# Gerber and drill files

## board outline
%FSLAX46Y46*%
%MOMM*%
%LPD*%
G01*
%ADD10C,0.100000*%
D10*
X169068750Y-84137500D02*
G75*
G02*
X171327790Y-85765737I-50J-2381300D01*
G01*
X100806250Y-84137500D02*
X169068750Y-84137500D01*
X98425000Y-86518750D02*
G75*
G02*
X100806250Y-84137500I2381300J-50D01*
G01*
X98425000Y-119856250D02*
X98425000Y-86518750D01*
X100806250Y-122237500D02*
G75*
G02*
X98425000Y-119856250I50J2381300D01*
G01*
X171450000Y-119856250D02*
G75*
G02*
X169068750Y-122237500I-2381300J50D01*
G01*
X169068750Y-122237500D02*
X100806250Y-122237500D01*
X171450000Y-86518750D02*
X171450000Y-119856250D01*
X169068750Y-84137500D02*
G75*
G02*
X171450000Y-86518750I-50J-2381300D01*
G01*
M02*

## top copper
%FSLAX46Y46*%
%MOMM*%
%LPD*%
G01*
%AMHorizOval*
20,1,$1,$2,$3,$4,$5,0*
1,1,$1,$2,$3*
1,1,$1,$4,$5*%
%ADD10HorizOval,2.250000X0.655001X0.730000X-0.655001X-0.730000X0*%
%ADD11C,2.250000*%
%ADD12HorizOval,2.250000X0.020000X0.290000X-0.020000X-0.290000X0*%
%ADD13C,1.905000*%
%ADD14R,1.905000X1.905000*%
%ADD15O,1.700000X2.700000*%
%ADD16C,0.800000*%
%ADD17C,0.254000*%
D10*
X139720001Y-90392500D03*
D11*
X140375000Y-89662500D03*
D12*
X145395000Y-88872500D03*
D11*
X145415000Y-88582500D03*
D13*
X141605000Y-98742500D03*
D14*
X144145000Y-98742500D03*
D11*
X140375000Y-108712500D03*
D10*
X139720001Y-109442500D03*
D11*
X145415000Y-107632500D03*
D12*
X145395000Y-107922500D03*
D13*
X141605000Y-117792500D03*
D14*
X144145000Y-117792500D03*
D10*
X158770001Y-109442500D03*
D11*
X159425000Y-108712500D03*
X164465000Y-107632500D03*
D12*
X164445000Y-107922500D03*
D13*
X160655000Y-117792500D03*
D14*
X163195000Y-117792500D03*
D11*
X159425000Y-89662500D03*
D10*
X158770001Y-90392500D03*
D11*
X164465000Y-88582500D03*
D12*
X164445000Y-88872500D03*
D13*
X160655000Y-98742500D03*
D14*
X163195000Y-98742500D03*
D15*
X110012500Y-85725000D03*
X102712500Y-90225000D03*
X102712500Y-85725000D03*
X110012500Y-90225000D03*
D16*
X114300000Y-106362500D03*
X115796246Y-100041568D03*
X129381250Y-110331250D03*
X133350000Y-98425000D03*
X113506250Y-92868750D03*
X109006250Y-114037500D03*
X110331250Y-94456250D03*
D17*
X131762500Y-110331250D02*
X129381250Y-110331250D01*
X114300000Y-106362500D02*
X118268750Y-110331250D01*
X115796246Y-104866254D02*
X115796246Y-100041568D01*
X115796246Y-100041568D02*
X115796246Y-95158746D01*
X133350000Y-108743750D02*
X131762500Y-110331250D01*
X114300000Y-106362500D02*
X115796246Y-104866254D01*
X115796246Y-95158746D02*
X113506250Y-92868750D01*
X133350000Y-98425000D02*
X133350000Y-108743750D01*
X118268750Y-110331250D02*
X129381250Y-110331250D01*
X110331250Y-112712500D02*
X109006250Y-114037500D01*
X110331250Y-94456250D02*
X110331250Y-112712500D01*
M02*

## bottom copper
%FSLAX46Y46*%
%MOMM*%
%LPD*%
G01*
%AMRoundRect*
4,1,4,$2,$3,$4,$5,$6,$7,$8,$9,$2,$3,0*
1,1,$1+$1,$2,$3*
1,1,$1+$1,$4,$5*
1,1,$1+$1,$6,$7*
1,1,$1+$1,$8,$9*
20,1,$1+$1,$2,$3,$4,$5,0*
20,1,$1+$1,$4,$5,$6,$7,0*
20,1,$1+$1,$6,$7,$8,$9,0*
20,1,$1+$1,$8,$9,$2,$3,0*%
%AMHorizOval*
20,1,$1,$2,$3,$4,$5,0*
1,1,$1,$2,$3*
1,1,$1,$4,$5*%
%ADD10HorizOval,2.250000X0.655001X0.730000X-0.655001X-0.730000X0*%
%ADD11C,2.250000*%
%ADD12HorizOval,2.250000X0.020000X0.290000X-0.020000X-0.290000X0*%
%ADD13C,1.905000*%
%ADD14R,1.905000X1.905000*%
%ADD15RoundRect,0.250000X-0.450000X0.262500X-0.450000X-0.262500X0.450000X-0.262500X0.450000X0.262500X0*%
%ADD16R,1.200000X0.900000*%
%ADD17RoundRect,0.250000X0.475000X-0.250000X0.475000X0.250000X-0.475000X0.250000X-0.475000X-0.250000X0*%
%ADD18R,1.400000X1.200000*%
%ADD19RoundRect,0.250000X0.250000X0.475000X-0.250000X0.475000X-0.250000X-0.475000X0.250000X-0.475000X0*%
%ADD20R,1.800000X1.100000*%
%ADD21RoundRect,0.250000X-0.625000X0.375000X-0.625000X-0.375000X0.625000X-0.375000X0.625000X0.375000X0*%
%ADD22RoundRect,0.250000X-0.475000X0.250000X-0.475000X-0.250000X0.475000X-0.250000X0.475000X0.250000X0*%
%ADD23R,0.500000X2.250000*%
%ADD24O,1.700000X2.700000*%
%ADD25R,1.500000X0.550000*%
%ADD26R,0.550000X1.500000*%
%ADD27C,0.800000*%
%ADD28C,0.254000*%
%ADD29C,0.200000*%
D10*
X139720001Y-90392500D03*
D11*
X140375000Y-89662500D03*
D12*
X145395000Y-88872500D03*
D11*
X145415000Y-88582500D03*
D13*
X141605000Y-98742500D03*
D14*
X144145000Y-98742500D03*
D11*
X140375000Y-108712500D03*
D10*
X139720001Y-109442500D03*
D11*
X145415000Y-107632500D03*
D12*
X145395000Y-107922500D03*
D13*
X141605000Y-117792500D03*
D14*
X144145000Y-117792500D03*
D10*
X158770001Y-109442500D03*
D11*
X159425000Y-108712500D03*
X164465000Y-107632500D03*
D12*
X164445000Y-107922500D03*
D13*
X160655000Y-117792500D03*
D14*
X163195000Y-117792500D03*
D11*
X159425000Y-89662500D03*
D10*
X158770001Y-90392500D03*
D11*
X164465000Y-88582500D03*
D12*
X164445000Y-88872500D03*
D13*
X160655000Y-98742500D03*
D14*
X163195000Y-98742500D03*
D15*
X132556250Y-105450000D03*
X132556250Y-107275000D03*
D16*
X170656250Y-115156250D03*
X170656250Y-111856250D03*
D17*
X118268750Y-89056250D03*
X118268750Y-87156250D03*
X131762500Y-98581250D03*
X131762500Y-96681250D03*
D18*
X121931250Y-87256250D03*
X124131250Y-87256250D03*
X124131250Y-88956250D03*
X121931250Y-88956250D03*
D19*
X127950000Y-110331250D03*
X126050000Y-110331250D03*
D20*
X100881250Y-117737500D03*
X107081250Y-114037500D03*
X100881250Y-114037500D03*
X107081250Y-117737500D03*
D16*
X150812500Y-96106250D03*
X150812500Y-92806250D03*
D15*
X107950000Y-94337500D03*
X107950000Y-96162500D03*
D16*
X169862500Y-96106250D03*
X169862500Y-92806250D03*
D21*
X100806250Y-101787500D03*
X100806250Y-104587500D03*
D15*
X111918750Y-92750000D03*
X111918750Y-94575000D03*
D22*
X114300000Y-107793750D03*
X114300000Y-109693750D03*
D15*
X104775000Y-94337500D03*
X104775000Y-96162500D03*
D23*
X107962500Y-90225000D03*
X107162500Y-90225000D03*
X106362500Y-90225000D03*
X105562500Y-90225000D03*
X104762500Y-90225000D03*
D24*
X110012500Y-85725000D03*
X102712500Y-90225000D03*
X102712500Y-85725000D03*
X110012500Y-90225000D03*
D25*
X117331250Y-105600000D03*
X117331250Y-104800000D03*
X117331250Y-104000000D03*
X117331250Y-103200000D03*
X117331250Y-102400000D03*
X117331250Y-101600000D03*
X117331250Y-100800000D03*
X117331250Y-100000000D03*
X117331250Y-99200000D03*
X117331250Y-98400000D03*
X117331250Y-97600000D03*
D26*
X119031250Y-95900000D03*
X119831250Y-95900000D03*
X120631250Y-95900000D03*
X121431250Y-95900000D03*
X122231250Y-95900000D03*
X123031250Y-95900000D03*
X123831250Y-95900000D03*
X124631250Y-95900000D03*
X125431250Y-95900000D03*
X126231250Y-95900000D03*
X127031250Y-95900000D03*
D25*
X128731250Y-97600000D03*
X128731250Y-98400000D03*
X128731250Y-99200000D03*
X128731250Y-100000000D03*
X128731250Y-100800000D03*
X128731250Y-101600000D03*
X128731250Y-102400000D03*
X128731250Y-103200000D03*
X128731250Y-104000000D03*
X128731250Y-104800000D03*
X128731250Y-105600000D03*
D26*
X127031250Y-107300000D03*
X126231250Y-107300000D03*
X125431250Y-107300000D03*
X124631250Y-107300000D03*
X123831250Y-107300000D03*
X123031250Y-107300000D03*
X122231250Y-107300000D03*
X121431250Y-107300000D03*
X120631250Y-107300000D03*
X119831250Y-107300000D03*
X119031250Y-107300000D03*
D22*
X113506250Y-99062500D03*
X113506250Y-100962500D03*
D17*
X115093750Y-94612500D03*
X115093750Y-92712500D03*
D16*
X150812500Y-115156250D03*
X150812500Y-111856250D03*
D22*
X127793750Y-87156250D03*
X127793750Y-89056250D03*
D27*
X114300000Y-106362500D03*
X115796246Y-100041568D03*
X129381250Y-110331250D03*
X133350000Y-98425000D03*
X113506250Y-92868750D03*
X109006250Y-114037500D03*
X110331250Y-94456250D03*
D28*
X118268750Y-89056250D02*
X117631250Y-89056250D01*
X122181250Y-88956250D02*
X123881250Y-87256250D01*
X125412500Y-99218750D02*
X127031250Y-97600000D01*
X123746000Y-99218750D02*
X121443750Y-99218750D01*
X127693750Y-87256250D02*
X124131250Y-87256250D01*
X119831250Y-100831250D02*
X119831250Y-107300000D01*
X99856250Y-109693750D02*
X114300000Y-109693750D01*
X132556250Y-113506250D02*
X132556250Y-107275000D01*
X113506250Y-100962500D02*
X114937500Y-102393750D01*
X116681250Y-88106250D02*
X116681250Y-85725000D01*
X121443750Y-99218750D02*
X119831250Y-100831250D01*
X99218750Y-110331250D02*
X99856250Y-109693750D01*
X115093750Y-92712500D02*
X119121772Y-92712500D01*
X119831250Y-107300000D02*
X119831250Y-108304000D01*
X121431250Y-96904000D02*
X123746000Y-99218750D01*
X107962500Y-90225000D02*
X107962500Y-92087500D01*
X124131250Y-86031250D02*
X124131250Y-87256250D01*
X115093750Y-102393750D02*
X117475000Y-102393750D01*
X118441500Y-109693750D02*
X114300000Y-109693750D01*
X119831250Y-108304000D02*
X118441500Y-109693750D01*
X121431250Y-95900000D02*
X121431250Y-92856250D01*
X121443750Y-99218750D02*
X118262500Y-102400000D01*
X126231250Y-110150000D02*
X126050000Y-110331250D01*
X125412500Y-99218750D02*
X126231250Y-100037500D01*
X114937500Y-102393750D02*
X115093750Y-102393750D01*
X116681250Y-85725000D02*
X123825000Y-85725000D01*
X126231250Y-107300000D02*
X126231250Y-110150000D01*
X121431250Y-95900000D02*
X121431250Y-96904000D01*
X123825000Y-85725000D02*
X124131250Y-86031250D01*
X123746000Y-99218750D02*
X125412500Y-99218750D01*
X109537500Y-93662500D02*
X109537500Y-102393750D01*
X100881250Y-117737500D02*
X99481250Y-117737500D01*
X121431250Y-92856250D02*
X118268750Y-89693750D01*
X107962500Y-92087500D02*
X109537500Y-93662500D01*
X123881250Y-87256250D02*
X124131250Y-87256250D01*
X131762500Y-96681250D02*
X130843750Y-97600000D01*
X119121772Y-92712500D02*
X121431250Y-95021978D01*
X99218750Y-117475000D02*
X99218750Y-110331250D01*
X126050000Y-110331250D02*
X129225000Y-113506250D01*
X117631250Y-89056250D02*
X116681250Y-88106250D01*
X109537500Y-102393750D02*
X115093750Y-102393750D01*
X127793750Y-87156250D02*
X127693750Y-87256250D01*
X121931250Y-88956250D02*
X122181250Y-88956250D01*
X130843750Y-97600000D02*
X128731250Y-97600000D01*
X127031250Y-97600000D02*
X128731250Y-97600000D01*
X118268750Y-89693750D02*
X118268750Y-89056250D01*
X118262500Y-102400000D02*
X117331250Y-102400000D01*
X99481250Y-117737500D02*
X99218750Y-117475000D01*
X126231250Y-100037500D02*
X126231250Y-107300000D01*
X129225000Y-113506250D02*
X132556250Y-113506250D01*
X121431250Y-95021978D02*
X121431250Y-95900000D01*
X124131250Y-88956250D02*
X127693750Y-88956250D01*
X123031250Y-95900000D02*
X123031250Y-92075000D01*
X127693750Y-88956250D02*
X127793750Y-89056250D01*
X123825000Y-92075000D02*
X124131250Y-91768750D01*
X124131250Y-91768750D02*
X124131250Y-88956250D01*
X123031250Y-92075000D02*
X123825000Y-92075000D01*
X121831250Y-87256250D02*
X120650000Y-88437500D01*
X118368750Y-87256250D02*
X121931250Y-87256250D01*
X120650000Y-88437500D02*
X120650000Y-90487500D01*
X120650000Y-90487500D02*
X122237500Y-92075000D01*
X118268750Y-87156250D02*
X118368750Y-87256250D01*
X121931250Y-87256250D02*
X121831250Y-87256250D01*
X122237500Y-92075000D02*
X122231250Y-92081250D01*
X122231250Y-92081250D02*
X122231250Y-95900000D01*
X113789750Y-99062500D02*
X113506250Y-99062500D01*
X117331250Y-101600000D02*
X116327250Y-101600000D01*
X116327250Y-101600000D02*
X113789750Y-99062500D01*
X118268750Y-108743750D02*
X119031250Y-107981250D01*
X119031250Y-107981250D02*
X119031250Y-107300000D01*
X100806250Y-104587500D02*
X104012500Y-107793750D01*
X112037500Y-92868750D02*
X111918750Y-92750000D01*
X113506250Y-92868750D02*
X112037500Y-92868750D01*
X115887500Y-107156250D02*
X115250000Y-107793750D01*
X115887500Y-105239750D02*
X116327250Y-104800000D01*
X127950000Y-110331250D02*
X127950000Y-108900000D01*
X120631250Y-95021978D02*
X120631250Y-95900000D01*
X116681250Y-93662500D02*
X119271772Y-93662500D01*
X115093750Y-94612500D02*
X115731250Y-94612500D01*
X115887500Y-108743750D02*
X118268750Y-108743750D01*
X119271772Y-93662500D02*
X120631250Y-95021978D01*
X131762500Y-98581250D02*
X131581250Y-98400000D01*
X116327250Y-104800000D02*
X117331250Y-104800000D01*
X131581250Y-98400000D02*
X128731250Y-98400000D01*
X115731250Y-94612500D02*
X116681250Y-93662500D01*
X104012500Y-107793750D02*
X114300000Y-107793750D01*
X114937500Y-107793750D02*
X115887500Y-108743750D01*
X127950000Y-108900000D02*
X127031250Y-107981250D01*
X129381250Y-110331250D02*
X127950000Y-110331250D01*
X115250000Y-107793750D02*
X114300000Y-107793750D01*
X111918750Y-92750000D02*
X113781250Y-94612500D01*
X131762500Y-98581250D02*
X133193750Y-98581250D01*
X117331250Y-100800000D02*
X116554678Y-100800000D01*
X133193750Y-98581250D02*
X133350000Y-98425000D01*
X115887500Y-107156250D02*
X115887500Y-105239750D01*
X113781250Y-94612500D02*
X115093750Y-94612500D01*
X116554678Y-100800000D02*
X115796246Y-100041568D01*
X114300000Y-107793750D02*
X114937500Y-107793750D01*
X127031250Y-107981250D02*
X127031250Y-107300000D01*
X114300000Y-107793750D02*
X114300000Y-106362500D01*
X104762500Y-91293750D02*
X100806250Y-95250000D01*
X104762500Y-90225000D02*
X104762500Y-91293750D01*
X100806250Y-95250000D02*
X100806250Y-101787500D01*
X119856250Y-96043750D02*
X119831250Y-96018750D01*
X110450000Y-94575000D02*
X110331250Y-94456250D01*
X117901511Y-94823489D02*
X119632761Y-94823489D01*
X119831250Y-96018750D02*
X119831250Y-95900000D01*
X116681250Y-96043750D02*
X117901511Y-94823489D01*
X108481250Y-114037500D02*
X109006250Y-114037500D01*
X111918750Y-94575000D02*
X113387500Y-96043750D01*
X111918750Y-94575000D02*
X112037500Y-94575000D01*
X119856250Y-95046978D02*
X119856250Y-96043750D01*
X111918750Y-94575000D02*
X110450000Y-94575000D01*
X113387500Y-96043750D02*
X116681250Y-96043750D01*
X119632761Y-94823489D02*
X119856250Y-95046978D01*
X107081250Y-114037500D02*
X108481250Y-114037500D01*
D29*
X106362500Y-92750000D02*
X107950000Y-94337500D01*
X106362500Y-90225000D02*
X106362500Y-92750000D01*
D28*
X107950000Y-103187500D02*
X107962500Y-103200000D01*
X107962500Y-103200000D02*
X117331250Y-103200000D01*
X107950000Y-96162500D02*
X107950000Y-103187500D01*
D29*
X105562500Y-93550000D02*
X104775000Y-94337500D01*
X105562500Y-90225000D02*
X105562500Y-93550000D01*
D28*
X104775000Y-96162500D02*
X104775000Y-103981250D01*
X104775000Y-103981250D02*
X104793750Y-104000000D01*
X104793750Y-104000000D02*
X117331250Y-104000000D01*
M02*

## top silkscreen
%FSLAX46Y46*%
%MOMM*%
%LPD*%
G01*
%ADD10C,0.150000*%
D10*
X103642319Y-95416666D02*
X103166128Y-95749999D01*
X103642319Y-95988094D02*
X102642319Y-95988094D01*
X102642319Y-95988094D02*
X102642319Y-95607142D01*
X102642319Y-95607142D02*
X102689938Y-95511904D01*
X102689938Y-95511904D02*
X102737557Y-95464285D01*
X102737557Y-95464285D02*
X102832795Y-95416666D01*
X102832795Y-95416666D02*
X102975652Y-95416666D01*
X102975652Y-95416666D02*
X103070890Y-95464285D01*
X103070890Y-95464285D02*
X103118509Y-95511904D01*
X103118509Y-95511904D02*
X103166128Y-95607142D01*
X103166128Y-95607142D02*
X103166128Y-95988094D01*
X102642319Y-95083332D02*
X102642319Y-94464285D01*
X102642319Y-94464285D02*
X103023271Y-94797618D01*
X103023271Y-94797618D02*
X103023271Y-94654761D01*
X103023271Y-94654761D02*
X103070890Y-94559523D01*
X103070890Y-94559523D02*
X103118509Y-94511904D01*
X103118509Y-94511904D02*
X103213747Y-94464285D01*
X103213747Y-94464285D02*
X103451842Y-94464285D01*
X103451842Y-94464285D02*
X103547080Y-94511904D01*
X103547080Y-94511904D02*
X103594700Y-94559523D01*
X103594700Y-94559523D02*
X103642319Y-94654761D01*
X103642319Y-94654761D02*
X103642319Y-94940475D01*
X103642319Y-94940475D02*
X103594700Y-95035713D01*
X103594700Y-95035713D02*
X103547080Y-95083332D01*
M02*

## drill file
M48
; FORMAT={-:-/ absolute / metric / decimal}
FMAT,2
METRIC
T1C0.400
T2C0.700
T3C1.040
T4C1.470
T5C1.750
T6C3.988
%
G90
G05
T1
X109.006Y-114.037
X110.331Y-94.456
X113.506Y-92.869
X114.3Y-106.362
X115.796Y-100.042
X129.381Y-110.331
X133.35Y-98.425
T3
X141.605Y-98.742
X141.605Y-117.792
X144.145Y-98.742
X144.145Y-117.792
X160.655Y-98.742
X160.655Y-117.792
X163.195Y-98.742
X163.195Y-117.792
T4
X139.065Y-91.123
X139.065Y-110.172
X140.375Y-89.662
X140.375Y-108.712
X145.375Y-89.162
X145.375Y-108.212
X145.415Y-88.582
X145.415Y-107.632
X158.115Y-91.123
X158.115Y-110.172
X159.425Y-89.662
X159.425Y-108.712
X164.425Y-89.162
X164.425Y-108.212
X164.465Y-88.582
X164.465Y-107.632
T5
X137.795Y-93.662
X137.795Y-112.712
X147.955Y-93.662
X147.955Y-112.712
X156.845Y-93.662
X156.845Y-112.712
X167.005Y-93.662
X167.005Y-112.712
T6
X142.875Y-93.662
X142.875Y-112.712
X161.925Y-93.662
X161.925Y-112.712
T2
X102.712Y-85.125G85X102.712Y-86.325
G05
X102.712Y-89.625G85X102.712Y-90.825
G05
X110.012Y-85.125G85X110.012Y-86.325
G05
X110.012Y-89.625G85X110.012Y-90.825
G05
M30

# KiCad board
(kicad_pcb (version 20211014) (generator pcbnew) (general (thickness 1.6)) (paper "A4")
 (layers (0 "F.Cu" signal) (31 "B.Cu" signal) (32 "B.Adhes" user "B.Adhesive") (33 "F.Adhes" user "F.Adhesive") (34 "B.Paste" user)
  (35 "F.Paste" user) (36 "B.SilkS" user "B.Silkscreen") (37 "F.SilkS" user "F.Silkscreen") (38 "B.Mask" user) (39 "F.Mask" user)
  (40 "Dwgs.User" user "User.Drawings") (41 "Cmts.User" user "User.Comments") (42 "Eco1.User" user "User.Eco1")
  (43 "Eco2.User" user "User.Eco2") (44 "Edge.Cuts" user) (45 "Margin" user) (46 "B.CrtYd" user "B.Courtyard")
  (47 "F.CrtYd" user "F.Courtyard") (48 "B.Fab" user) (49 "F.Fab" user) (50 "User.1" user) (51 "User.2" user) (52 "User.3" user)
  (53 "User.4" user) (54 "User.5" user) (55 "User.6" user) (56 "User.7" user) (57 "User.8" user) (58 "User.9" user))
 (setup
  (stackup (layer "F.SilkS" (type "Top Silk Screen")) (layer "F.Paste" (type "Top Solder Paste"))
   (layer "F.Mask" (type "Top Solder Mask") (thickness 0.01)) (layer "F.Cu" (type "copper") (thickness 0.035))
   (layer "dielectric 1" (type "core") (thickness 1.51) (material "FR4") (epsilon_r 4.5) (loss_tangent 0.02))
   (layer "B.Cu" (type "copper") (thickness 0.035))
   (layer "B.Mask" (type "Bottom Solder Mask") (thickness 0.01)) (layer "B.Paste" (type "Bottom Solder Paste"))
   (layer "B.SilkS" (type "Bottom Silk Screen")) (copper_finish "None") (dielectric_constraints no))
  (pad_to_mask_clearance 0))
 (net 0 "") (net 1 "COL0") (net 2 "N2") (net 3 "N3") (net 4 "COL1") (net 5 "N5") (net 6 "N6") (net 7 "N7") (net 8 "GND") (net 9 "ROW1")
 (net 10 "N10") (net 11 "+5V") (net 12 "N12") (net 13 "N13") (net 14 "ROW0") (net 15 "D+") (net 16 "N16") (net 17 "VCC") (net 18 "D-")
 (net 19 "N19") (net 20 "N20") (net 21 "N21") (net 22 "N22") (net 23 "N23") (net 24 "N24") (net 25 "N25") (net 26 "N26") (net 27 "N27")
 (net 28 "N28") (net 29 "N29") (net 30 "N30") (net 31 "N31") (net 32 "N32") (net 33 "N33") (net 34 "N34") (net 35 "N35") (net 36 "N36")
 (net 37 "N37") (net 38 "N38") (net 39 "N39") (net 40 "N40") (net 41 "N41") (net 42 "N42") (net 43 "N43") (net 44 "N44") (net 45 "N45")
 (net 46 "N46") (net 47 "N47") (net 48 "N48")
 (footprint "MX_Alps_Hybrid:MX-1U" (layer "F.Cu") (at 142.875 93.6625)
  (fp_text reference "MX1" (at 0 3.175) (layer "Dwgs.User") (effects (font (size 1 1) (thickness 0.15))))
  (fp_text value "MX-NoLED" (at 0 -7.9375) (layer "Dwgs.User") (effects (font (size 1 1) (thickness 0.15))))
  (pad "" np_thru_hole circle locked (at 5.08 0 48.0996) (size 1.75 1.75) (drill 1.75) (layers *.Cu *.Mask))
  (pad "" np_thru_hole circle locked (at 0 0) (size 3.9878 3.9878) (drill 3.9878) (layers *.Cu *.Mask))
  (pad "" np_thru_hole circle locked (at -5.08 0 48.0996) (size 1.75 1.75) (drill 1.75) (layers *.Cu *.Mask))
  (pad "1" thru_hole oval locked (at -3.81 -2.54 48.0996) (size 4.211556 2.25) (drill 1.47 (offset 0.980778 0)) (layers *.Cu "B.Mask")
   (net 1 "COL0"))
  (pad "1" thru_hole circle locked (at -2.5 -4) (size 2.25 2.25) (drill 1.47) (layers *.Cu "B.Mask") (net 1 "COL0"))
  (pad "2" thru_hole oval locked (at 2.5 -4.5 86.0548) (size 2.831378 2.25) (drill 1.47 (offset 0.290689 0)) (layers *.Cu "B.Mask")
   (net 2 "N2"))
  (pad "2" thru_hole circle locked (at 2.54 -5.08) (size 2.25 2.25) (drill 1.47) (layers *.Cu "B.Mask") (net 2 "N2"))
  (pad "3" thru_hole circle locked (at -1.27 5.08) (size 1.905 1.905) (drill 1.04) (layers *.Cu "B.Mask"))
  (pad "4" thru_hole rect locked (at 1.27 5.08) (size 1.905 1.905) (drill 1.04) (layers *.Cu "B.Mask")))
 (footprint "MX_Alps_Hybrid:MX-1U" (layer "F.Cu") (at 142.875 112.7125)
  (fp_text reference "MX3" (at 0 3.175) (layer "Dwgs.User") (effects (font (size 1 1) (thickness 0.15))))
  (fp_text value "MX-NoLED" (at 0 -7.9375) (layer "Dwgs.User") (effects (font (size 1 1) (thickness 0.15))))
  (pad "" np_thru_hole circle locked (at -5.08 0 48.0996) (size 1.75 1.75) (drill 1.75) (layers *.Cu *.Mask))
  (pad "" np_thru_hole circle locked (at 0 0) (size 3.9878 3.9878) (drill 3.9878) (layers *.Cu *.Mask))
  (pad "" np_thru_hole circle locked (at 5.08 0 48.0996) (size 1.75 1.75) (drill 1.75) (layers *.Cu *.Mask))
  (pad "1" thru_hole circle locked (at -2.5 -4) (size 2.25 2.25) (drill 1.47) (layers *.Cu "B.Mask") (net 1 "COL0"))
  (pad "1" thru_hole oval locked (at -3.81 -2.54 48.0996) (size 4.211556 2.25) (drill 1.47 (offset 0.980778 0)) (layers *.Cu "B.Mask")
   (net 1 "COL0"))
  (pad "2" thru_hole circle locked (at 2.54 -5.08) (size 2.25 2.25) (drill 1.47) (layers *.Cu "B.Mask") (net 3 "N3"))
  (pad "2" thru_hole oval locked (at 2.5 -4.5 86.0548) (size 2.831378 2.25) (drill 1.47 (offset 0.290689 0)) (layers *.Cu "B.Mask")
   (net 3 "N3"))
  (pad "3" thru_hole circle locked (at -1.27 5.08) (size 1.905 1.905) (drill 1.04) (layers *.Cu "B.Mask"))
  (pad "4" thru_hole rect locked (at 1.27 5.08) (size 1.905 1.905) (drill 1.04) (layers *.Cu "B.Mask")))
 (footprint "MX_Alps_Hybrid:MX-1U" (layer "F.Cu") (at 161.925 112.7125)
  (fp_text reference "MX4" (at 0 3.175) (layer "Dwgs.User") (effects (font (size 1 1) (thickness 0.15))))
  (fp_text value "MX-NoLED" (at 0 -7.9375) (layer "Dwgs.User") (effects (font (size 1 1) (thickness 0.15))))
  (pad "" np_thru_hole circle locked (at 0 0) (size 3.9878 3.9878) (drill 3.9878) (layers *.Cu *.Mask))
  (pad "" np_thru_hole circle locked (at 5.08 0 48.0996) (size 1.75 1.75) (drill 1.75) (layers *.Cu *.Mask))
  (pad "" np_thru_hole circle locked (at -5.08 0 48.0996) (size 1.75 1.75) (drill 1.75) (layers *.Cu *.Mask))
  (pad "1" thru_hole oval locked (at -3.81 -2.54 48.0996) (size 4.211556 2.25) (drill 1.47 (offset 0.980778 0)) (layers *.Cu "B.Mask")
   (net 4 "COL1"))
  (pad "1" thru_hole circle locked (at -2.5 -4) (size 2.25 2.25) (drill 1.47) (layers *.Cu "B.Mask") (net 4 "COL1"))
  (pad "2" thru_hole circle locked (at 2.54 -5.08) (size 2.25 2.25) (drill 1.47) (layers *.Cu "B.Mask") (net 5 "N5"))
  (pad "2" thru_hole oval locked (at 2.5 -4.5 86.0548) (size 2.831378 2.25) (drill 1.47 (offset 0.290689 0)) (layers *.Cu "B.Mask")
   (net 5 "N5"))
  (pad "3" thru_hole circle locked (at -1.27 5.08) (size 1.905 1.905) (drill 1.04) (layers *.Cu "B.Mask"))
  (pad "4" thru_hole rect locked (at 1.27 5.08) (size 1.905 1.905) (drill 1.04) (layers *.Cu "B.Mask")))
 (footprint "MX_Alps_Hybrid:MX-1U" (layer "F.Cu") (at 161.925 93.6625)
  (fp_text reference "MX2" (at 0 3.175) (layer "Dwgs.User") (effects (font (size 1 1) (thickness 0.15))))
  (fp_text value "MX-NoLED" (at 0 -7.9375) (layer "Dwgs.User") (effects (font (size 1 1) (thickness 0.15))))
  (pad "" np_thru_hole circle locked (at 0 0) (size 3.9878 3.9878) (drill 3.9878) (layers *.Cu *.Mask))
  (pad "" np_thru_hole circle locked (at 5.08 0 48.0996) (size 1.75 1.75) (drill 1.75) (layers *.Cu *.Mask))
  (pad "" np_thru_hole circle locked (at -5.08 0 48.0996) (size 1.75 1.75) (drill 1.75) (layers *.Cu *.Mask))
  (pad "1" thru_hole circle locked (at -2.5 -4) (size 2.25 2.25) (drill 1.47) (layers *.Cu "B.Mask") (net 4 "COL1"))
  (pad "1" thru_hole oval locked (at -3.81 -2.54 48.0996) (size 4.211556 2.25) (drill 1.47 (offset 0.980778 0)) (layers *.Cu "B.Mask")
   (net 4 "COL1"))
  (pad "2" thru_hole circle locked (at 2.54 -5.08) (size 2.25 2.25) (drill 1.47) (layers *.Cu "B.Mask") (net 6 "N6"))
  (pad "2" thru_hole oval locked (at 2.5 -4.5 86.0548) (size 2.831378 2.25) (drill 1.47 (offset 0.290689 0)) (layers *.Cu "B.Mask")
   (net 6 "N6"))
  (pad "3" thru_hole circle locked (at -1.27 5.08) (size 1.905 1.905) (drill 1.04) (layers *.Cu "B.Mask"))
  (pad "4" thru_hole rect locked (at 1.27 5.08) (size 1.905 1.905) (drill 1.04) (layers *.Cu "B.Mask")))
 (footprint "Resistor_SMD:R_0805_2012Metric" (layer "B.Cu") (at 132.55625 106.3625 -90)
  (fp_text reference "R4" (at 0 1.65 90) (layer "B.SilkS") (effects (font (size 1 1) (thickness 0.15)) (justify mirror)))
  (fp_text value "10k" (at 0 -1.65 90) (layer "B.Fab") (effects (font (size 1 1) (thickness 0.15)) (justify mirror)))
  (pad "1" smd roundrect (at -0.9125 0 270) (size 1.025 1.4) (layers "B.Cu" "B.Paste" "B.Mask") (roundrect_rratio 0.243902) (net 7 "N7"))
  (pad "2" smd roundrect (at 0.9125 0 270) (size 1.025 1.4) (layers "B.Cu" "B.Paste" "B.Mask") (roundrect_rratio 0.243902) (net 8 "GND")))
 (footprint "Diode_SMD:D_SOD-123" (layer "B.Cu") (at 170.65625 113.50625 90)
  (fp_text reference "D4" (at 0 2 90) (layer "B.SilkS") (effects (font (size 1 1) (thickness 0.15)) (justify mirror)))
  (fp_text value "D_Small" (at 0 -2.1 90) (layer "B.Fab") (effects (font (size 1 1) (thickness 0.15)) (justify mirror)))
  (pad "1" smd rect (at -1.65 0 90) (size 0.9 1.2) (layers "B.Cu" "B.Paste" "B.Mask") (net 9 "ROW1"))
  (pad "2" smd rect (at 1.65 0 90) (size 0.9 1.2) (layers "B.Cu" "B.Paste" "B.Mask") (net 5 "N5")))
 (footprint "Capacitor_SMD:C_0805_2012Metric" (layer "B.Cu") (at 118.26875 88.10625 90)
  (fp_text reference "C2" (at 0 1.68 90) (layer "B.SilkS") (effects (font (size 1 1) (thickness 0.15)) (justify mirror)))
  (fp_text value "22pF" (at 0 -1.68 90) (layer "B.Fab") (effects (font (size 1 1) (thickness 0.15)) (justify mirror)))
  (pad "1" smd roundrect (at -0.95 0 90) (size 1 1.45) (layers "B.Cu" "B.Paste" "B.Mask") (roundrect_rratio 0.25) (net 8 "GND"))
  (pad "2" smd roundrect (at 0.95 0 90) (size 1 1.45) (layers "B.Cu" "B.Paste" "B.Mask") (roundrect_rratio 0.25) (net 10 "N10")))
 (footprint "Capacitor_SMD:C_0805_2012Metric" (layer "B.Cu") (at 131.7625 97.63125 90)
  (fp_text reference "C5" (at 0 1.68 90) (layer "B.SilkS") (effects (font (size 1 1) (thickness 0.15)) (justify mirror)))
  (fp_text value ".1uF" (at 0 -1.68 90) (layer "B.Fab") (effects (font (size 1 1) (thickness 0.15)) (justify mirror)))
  (pad "1" smd roundrect (at -0.95 0 90) (size 1 1.45) (layers "B.Cu" "B.Paste" "B.Mask") (roundrect_rratio 0.25) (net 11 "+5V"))
  (pad "2" smd roundrect (at 0.95 0 90) (size 1 1.45) (layers "B.Cu" "B.Paste" "B.Mask") (roundrect_rratio 0.25) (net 8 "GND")))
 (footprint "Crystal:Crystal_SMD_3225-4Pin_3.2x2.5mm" (layer "B.Cu") (at 123.03125 88.10625)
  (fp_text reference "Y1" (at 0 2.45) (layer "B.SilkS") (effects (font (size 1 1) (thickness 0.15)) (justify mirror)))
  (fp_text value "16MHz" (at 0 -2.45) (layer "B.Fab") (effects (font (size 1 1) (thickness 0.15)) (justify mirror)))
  (pad "1" smd rect (at -1.1 -0.85) (size 1.4 1.2) (layers "B.Cu" "B.Paste" "B.Mask") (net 10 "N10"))
  (pad "2" smd rect (at 1.1 -0.85) (size 1.4 1.2) (layers "B.Cu" "B.Paste" "B.Mask") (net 8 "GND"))
  (pad "3" smd rect (at 1.1 0.85) (size 1.4 1.2) (layers "B.Cu" "B.Paste" "B.Mask") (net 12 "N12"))
  (pad "4" smd rect (at -1.1 0.85) (size 1.4 1.2) (layers "B.Cu" "B.Paste" "B.Mask") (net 8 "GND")))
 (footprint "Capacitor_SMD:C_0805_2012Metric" (layer "B.Cu") (at 127 110.33125 180)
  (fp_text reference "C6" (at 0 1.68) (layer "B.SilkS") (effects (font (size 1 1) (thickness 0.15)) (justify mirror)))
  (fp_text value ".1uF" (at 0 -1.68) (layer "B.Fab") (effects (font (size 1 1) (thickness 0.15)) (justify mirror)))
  (pad "1" smd roundrect (at -0.95 0 180) (size 1 1.45) (layers "B.Cu" "B.Paste" "B.Mask") (roundrect_rratio 0.25) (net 11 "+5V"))
  (pad "2" smd roundrect (at 0.95 0 180) (size 1 1.45) (layers "B.Cu" "B.Paste" "B.Mask") (roundrect_rratio 0.25) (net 8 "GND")))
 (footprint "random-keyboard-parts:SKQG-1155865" (layer "B.Cu") (at 103.98125 115.8875 180)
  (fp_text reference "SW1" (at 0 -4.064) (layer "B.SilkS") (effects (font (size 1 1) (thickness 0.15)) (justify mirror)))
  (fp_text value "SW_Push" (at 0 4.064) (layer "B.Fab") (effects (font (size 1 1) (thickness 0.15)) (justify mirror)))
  (pad "1" smd rect locked (at 3.1 -1.85 180) (size 1.8 1.1) (layers "B.Cu" "B.Paste" "B.Mask") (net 8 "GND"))
  (pad "2" smd rect locked (at -3.1 1.85 180) (size 1.8 1.1) (layers "B.Cu" "B.Paste" "B.Mask") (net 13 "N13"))
  (pad "3" smd rect locked (at 3.1 1.85 180) (size 1.8 1.1) (layers "B.Cu" "B.Paste" "B.Mask"))
  (pad "4" smd rect locked (at -3.1 -1.85 180) (size 1.8 1.1) (layers "B.Cu" "B.Paste" "B.Mask")))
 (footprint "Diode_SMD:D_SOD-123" (layer "B.Cu") (at 150.8125 94.45625 90)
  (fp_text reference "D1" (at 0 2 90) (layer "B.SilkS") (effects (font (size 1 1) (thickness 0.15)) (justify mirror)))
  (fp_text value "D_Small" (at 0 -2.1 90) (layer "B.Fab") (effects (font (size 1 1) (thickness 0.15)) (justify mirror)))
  (pad "1" smd rect (at -1.65 0 90) (size 0.9 1.2) (layers "B.Cu" "B.Paste" "B.Mask") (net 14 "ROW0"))
  (pad "2" smd rect (at 1.65 0 90) (size 0.9 1.2) (layers "B.Cu" "B.Paste" "B.Mask") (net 2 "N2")))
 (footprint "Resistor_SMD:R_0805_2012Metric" (layer "B.Cu") (at 107.95 95.25 -90)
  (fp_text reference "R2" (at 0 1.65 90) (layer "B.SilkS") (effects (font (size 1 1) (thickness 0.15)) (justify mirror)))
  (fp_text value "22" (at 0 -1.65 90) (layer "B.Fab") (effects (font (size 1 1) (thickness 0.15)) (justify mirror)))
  (pad "1" smd roundrect (at -0.9125 0 270) (size 1.025 1.4) (layers "B.Cu" "B.Paste" "B.Mask") (roundrect_rratio 0.243902) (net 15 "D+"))
  (pad "2" smd roundrect (at 0.9125 0 270) (size 1.025 1.4) (layers "B.Cu" "B.Paste" "B.Mask") (roundrect_rratio 0.243902) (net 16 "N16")))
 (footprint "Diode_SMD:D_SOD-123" (layer "B.Cu") (at 169.8625 94.45625 90)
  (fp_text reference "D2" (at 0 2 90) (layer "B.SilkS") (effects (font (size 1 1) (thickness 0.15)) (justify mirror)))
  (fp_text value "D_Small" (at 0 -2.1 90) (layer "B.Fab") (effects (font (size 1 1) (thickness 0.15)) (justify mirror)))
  (pad "1" smd rect (at -1.65 0 90) (size 0.9 1.2) (layers "B.Cu" "B.Paste" "B.Mask") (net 14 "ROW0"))
  (pad "2" smd rect (at 1.65 0 90) (size 0.9 1.2) (layers "B.Cu" "B.Paste" "B.Mask") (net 6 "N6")))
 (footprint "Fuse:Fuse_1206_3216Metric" (layer "B.Cu") (at 100.80625 103.1875 -90)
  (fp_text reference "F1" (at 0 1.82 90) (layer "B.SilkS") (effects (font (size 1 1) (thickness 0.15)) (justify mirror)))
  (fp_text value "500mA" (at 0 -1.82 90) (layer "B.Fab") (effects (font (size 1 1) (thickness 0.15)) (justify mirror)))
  (pad "1" smd roundrect (at -1.4 0 270) (size 1.25 1.75) (layers "B.Cu" "B.Paste" "B.Mask") (roundrect_rratio 0.2) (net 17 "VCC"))
  (pad "2" smd roundrect (at 1.4 0 270) (size 1.25 1.75) (layers "B.Cu" "B.Paste" "B.Mask") (roundrect_rratio 0.2) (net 11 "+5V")))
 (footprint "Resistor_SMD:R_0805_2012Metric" (layer "B.Cu") (at 111.91875 93.6625 -90)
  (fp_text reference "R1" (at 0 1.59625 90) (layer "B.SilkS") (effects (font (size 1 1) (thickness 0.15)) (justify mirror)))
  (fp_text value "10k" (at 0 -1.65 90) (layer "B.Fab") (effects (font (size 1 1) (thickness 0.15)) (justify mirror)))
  (pad "1" smd roundrect (at -0.9125 0 270) (size 1.025 1.4) (layers "B.Cu" "B.Paste" "B.Mask") (roundrect_rratio 0.243902) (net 11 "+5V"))
  (pad "2" smd roundrect (at 0.9125 0 270) (size 1.025 1.4) (layers "B.Cu" "B.Paste" "B.Mask") (roundrect_rratio 0.243902) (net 13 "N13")))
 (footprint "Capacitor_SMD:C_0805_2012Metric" (layer "B.Cu") (at 114.3 108.74375 -90)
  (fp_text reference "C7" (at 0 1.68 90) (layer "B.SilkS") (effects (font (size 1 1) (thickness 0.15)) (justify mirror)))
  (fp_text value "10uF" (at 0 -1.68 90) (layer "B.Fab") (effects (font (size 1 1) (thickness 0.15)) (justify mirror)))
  (pad "1" smd roundrect (at -0.95 0 270) (size 1 1.45) (layers "B.Cu" "B.Paste" "B.Mask") (roundrect_rratio 0.25) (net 11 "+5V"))
  (pad "2" smd roundrect (at 0.95 0 270) (size 1 1.45) (layers "B.Cu" "B.Paste" "B.Mask") (roundrect_rratio 0.25) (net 8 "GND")))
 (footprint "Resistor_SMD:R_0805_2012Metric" (layer "B.Cu") (at 104.775 95.25 -90)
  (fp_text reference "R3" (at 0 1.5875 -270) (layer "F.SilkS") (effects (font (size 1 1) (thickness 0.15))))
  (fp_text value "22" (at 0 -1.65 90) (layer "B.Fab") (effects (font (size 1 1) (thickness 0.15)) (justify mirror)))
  (pad "1" smd roundrect (at -0.9125 0 270) (size 1.025 1.4) (layers "B.Cu" "B.Paste" "B.Mask") (roundrect_rratio 0.243902) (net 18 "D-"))
  (pad "2" smd roundrect (at 0.9125 0 270) (size 1.025 1.4) (layers "B.Cu" "B.Paste" "B.Mask") (roundrect_rratio 0.243902) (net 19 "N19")))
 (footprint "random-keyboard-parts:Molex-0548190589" (layer "B.Cu") (at 106.3625 85.725 -90)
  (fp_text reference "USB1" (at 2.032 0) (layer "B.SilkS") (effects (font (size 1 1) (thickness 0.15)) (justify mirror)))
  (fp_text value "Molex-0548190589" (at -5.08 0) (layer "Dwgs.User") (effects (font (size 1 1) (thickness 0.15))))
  (pad "1" smd rect locked (at 4.5 -1.6 270) (size 2.25 0.5) (layers "B.Cu" "B.Paste" "B.Mask") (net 8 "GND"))
  (pad "2" smd rect locked (at 4.5 -0.8 270) (size 2.25 0.5) (layers "B.Cu" "B.Paste" "B.Mask") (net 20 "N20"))
  (pad "3" smd rect locked (at 4.5 0 270) (size 2.25 0.5) (layers "B.Cu" "B.Paste" "B.Mask") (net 15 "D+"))
  (pad "4" smd rect locked (at 4.5 0.8 270) (size 2.25 0.5) (layers "B.Cu" "B.Paste" "B.Mask") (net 18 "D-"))
  (pad "5" smd rect locked (at 4.5 1.6 270) (size 2.25 0.5) (layers "B.Cu" "B.Paste" "B.Mask") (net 17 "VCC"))
  (pad "6" thru_hole oval locked (at 0 -3.65 270) (size 2.7 1.7) (drill oval 1.9 0.7) (layers *.Cu *.Mask) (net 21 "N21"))
  (pad "6" thru_hole oval locked (at 4.5 3.65 270) (size 2.7 1.7) (drill oval 1.9 0.7) (layers *.Cu *.Mask) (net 21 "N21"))
  (pad "6" thru_hole oval locked (at 0 3.65 270) (size 2.7 1.7) (drill oval 1.9 0.7) (layers *.Cu *.Mask) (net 21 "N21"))
  (pad "6" thru_hole oval locked (at 4.5 -3.65 270) (size 2.7 1.7) (drill oval 1.9 0.7) (layers *.Cu *.Mask) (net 21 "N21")))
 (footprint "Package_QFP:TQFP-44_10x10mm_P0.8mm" (layer "B.Cu") (at 123.03125 101.6)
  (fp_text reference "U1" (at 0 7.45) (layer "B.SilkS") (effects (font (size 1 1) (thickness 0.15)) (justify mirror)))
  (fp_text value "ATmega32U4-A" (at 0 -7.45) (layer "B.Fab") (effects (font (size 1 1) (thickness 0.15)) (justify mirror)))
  (pad "1" smd rect (at -5.7 4) (size 1.5 0.55) (layers "B.Cu" "B.Paste" "B.Mask") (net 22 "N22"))
  (pad "2" smd rect (at -5.7 3.2) (size 1.5 0.55) (layers "B.Cu" "B.Paste" "B.Mask") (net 11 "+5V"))
  (pad "3" smd rect (at -5.7 2.4) (size 1.5 0.55) (layers "B.Cu" "B.Paste" "B.Mask") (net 19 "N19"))
  (pad "4" smd rect (at -5.7 1.6) (size 1.5 0.55) (layers "B.Cu" "B.Paste" "B.Mask") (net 16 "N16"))
  (pad "5" smd rect (at -5.7 0.8) (size 1.5 0.55) (layers "B.Cu" "B.Paste" "B.Mask") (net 8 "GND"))
  (pad "6" smd rect (at -5.7 0) (size 1.5 0.55) (layers "B.Cu" "B.Paste" "B.Mask") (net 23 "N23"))
  (pad "7" smd rect (at -5.7 -0.8) (size 1.5 0.55) (layers "B.Cu" "B.Paste" "B.Mask") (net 11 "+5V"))
  (pad "8" smd rect (at -5.7 -1.6) (size 1.5 0.55) (layers "B.Cu" "B.Paste" "B.Mask") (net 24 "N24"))
  (pad "9" smd rect (at -5.7 -2.4) (size 1.5 0.55) (layers "B.Cu" "B.Paste" "B.Mask") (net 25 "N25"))
  (pad "10" smd rect (at -5.7 -3.2) (size 1.5 0.55) (layers "B.Cu" "B.Paste" "B.Mask") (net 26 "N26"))
  (pad "11" smd rect (at -5.7 -4) (size 1.5 0.55) (layers "B.Cu" "B.Paste" "B.Mask") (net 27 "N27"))
  (pad "12" smd rect (at -4 -5.7 270) (size 1.5 0.55) (layers "B.Cu" "B.Paste" "B.Mask") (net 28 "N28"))
  (pad "13" smd rect (at -3.2 -5.7 270) (size 1.5 0.55) (layers "B.Cu" "B.Paste" "B.Mask") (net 13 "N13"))
  (pad "14" smd rect (at -2.4 -5.7 270) (size 1.5 0.55) (layers "B.Cu" "B.Paste" "B.Mask") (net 11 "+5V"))
  (pad "15" smd rect (at -1.6 -5.7 270) (size 1.5 0.55) (layers "B.Cu" "B.Paste" "B.Mask") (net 8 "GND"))
  (pad "16" smd rect (at -0.8 -5.7 270) (size 1.5 0.55) (layers "B.Cu" "B.Paste" "B.Mask") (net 10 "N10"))
  (pad "17" smd rect (at 0 -5.7 270) (size 1.5 0.55) (layers "B.Cu" "B.Paste" "B.Mask") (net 12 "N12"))
  (pad "18" smd rect (at 0.8 -5.7 270) (size 1.5 0.55) (layers "B.Cu" "B.Paste" "B.Mask") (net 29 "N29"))
  (pad "19" smd rect (at 1.6 -5.7 270) (size 1.5 0.55) (layers "B.Cu" "B.Paste" "B.Mask") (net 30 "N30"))
  (pad "20" smd rect (at 2.4 -5.7 270) (size 1.5 0.55) (layers "B.Cu" "B.Paste" "B.Mask") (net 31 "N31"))
  (pad "21" smd rect (at 3.2 -5.7 270) (size 1.5 0.55) (layers "B.Cu" "B.Paste" "B.Mask") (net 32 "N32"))
  (pad "22" smd rect (at 4 -5.7 270) (size 1.5 0.55) (layers "B.Cu" "B.Paste" "B.Mask") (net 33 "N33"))
  (pad "23" smd rect (at 5.7 -4) (size 1.5 0.55) (layers "B.Cu" "B.Paste" "B.Mask") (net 8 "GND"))
  (pad "24" smd rect (at 5.7 -3.2) (size 1.5 0.55) (layers "B.Cu" "B.Paste" "B.Mask") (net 11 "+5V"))
  (pad "25" smd rect (at 5.7 -2.4) (size 1.5 0.55) (layers "B.Cu" "B.Paste" "B.Mask") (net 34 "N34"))
  (pad "26" smd rect (at 5.7 -1.6) (size 1.5 0.55) (layers "B.Cu" "B.Paste" "B.Mask") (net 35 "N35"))
  (pad "27" smd rect (at 5.7 -0.8) (size 1.5 0.55) (layers "B.Cu" "B.Paste" "B.Mask") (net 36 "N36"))
  (pad "28" smd rect (at 5.7 0) (size 1.5 0.55) (layers "B.Cu" "B.Paste" "B.Mask") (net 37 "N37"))
  (pad "29" smd rect (at 5.7 0.8) (size 1.5 0.55) (layers "B.Cu" "B.Paste" "B.Mask") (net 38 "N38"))
  (pad "30" smd rect (at 5.7 1.6) (size 1.5 0.55) (layers "B.Cu" "B.Paste" "B.Mask") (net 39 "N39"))
  (pad "31" smd rect (at 5.7 2.4) (size 1.5 0.55) (layers "B.Cu" "B.Paste" "B.Mask") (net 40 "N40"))
  (pad "32" smd rect (at 5.7 3.2) (size 1.5 0.55) (layers "B.Cu" "B.Paste" "B.Mask") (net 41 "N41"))
  (pad "33" smd rect (at 5.7 4) (size 1.5 0.55) (layers "B.Cu" "B.Paste" "B.Mask") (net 7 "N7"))
  (pad "34" smd rect (at 4 5.7 270) (size 1.5 0.55) (layers "B.Cu" "B.Paste" "B.Mask") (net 11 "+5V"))
  (pad "35" smd rect (at 3.2 5.7 270) (size 1.5 0.55) (layers "B.Cu" "B.Paste" "B.Mask") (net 8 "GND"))
  (pad "36" smd rect (at 2.4 5.7 270) (size 1.5 0.55) (layers "B.Cu" "B.Paste" "B.Mask") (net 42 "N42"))
  (pad "37" smd rect (at 1.6 5.7 270) (size 1.5 0.55) (layers "B.Cu" "B.Paste" "B.Mask") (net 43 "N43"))
  (pad "38" smd rect (at 0.8 5.7 270) (size 1.5 0.55) (layers "B.Cu" "B.Paste" "B.Mask") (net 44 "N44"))
  (pad "39" smd rect (at 0 5.7 270) (size 1.5 0.55) (layers "B.Cu" "B.Paste" "B.Mask") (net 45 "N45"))
  (pad "40" smd rect (at -0.8 5.7 270) (size 1.5 0.55) (layers "B.Cu" "B.Paste" "B.Mask") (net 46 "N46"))
  (pad "41" smd rect (at -1.6 5.7 270) (size 1.5 0.55) (layers "B.Cu" "B.Paste" "B.Mask") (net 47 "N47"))
  (pad "42" smd rect (at -2.4 5.7 270) (size 1.5 0.55) (layers "B.Cu" "B.Paste" "B.Mask") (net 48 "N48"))
  (pad "43" smd rect (at -3.2 5.7 270) (size 1.5 0.55) (layers "B.Cu" "B.Paste" "B.Mask") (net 8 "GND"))
  (pad "44" smd rect (at -4 5.7 270) (size 1.5 0.55) (layers "B.Cu" "B.Paste" "B.Mask") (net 11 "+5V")))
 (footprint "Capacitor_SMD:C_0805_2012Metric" (layer "B.Cu") (at 113.50625 100.0125 -90)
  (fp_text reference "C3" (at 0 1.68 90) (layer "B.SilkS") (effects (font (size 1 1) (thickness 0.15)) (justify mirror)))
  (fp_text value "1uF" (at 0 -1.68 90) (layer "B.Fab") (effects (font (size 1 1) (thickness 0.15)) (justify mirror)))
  (pad "1" smd roundrect (at -0.95 0 270) (size 1 1.45) (layers "B.Cu" "B.Paste" "B.Mask") (roundrect_rratio 0.25) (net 23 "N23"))
  (pad "2" smd roundrect (at 0.95 0 270) (size 1 1.45) (layers "B.Cu" "B.Paste" "B.Mask") (roundrect_rratio 0.25) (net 8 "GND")))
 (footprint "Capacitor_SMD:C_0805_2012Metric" (layer "B.Cu") (at 115.09375 93.6625 90)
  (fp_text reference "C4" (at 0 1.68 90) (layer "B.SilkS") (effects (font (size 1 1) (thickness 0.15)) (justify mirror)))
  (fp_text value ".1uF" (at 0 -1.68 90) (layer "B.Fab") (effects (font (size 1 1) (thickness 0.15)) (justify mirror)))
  (pad "1" smd roundrect (at -0.95 0 90) (size 1 1.45) (layers "B.Cu" "B.Paste" "B.Mask") (roundrect_rratio 0.25) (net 11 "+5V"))
  (pad "2" smd roundrect (at 0.95 0 90) (size 1 1.45) (layers "B.Cu" "B.Paste" "B.Mask") (roundrect_rratio 0.25) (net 8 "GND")))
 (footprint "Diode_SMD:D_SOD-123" (layer "B.Cu") (at 150.8125 113.50625 90)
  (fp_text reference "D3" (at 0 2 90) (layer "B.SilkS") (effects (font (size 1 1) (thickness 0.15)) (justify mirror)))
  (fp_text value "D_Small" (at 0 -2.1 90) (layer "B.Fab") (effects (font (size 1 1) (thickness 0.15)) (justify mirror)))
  (pad "1" smd rect (at -1.65 0 90) (size 0.9 1.2) (layers "B.Cu" "B.Paste" "B.Mask") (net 9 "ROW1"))
  (pad "2" smd rect (at 1.65 0 90) (size 0.9 1.2) (layers "B.Cu" "B.Paste" "B.Mask") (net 3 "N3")))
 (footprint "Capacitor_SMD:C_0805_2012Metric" (layer "B.Cu") (at 127.79375 88.10625 -90)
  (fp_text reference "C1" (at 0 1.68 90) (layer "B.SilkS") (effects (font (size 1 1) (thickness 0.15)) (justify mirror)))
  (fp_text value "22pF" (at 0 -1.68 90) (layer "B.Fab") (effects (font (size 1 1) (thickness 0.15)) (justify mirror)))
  (pad "1" smd roundrect (at -0.95 0 270) (size 1 1.45) (layers "B.Cu" "B.Paste" "B.Mask") (roundrect_rratio 0.25) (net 8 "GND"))
  (pad "2" smd roundrect (at 0.95 0 270) (size 1 1.45) (layers "B.Cu" "B.Paste" "B.Mask") (roundrect_rratio 0.25) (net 12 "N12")))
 (gr_arc (start 169.06875 84.1375) (mid 170.461091 84.58698) (end 171.327802 85.765733) (layer "Edge.Cuts") (width 0.1))
 (gr_line (start 100.80625 84.1375) (end 169.06875 84.1375) (layer "Edge.Cuts") (width 0.1))
 (gr_arc (start 98.425 86.51875) (mid 99.122452 84.834952) (end 100.80625 84.1375) (layer "Edge.Cuts") (width 0.1))
 (gr_line (start 98.425 119.85625) (end 98.425 86.51875) (layer "Edge.Cuts") (width 0.1))
 (gr_arc (start 100.80625 122.2375) (mid 99.122452 121.540048) (end 98.425 119.85625) (layer "Edge.Cuts") (width 0.1))
 (gr_arc (start 171.45 119.85625) (mid 170.752548 121.540048) (end 169.06875 122.2375) (layer "Edge.Cuts") (width 0.1))
 (gr_line (start 169.06875 122.2375) (end 100.80625 122.2375) (layer "Edge.Cuts") (width 0.1))
 (gr_line (start 171.45 86.51875) (end 171.45 119.85625) (layer "Edge.Cuts") (width 0.1))
 (gr_arc (start 169.06875 84.1375) (mid 170.752548 84.834952) (end 171.45 86.51875) (layer "Edge.Cuts") (width 0.1))
 (segment (start 118.26875 89.05625) (end 117.63125 89.05625) (width 0.254) (layer "B.Cu") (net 8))
 (segment (start 122.18125 88.95625) (end 123.88125 87.25625) (width 0.254) (layer "B.Cu") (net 8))
 (segment (start 125.4125 99.21875) (end 127.03125 97.6) (width 0.254) (layer "B.Cu") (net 8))
 (segment (start 123.746 99.21875) (end 121.44375 99.21875) (width 0.254) (layer "B.Cu") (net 8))
 (segment (start 127.69375 87.25625) (end 124.13125 87.25625) (width 0.254) (layer "B.Cu") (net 8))
 (segment (start 119.83125 100.83125) (end 119.83125 107.3) (width 0.254) (layer "B.Cu") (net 8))
 (segment (start 99.85625 109.69375) (end 114.3 109.69375) (width 0.254) (layer "B.Cu") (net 8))
 (segment (start 132.55625 113.50625) (end 132.55625 107.275) (width 0.254) (layer "B.Cu") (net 8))
 (segment (start 113.50625 100.9625) (end 114.9375 102.39375) (width 0.254) (layer "B.Cu") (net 8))
 (segment (start 116.68125 88.10625) (end 116.68125 85.725) (width 0.254) (layer "B.Cu") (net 8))
 (segment (start 121.44375 99.21875) (end 119.83125 100.83125) (width 0.254) (layer "B.Cu") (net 8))
 (segment (start 99.21875 110.33125) (end 99.85625 109.69375) (width 0.254) (layer "B.Cu") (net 8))
 (segment (start 115.09375 92.7125) (end 119.121772 92.7125) (width 0.254) (layer "B.Cu") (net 8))
 (segment (start 119.83125 107.3) (end 119.83125 108.304) (width 0.254) (layer "B.Cu") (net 8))
 (segment (start 121.43125 96.904) (end 123.746 99.21875) (width 0.254) (layer "B.Cu") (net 8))
 (segment (start 107.9625 90.225) (end 107.9625 92.0875) (width 0.254) (layer "B.Cu") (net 8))
 (segment (start 124.13125 86.03125) (end 124.13125 87.25625) (width 0.254) (layer "B.Cu") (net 8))
 (segment (start 115.09375 102.39375) (end 117.475 102.39375) (width 0.254) (layer "B.Cu") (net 8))
 (segment (start 118.4415 109.69375) (end 114.3 109.69375) (width 0.254) (layer "B.Cu") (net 8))
 (segment (start 119.83125 108.304) (end 118.4415 109.69375) (width 0.254) (layer "B.Cu") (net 8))
 (segment (start 121.43125 95.9) (end 121.43125 92.85625) (width 0.254) (layer "B.Cu") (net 8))
 (segment (start 121.44375 99.21875) (end 118.2625 102.4) (width 0.254) (layer "B.Cu") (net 8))
 (segment (start 126.23125 110.15) (end 126.05 110.33125) (width 0.254) (layer "B.Cu") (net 8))
 (segment (start 125.4125 99.21875) (end 126.23125 100.0375) (width 0.254) (layer "B.Cu") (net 8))
 (segment (start 114.9375 102.39375) (end 115.09375 102.39375) (width 0.254) (layer "B.Cu") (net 8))
 (segment (start 116.68125 85.725) (end 123.825 85.725) (width 0.254) (layer "B.Cu") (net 8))
 (segment (start 126.23125 107.3) (end 126.23125 110.15) (width 0.254) (layer "B.Cu") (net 8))
 (segment (start 121.43125 95.9) (end 121.43125 96.904) (width 0.254) (layer "B.Cu") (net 8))
 (segment (start 123.825 85.725) (end 124.13125 86.03125) (width 0.254) (layer "B.Cu") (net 8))
 (segment (start 123.746 99.21875) (end 125.4125 99.21875) (width 0.254) (layer "B.Cu") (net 8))
 (segment (start 109.5375 93.6625) (end 109.5375 102.39375) (width 0.254) (layer "B.Cu") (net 8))
 (segment (start 100.88125 117.7375) (end 99.48125 117.7375) (width 0.254) (layer "B.Cu") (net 8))
 (segment (start 121.43125 92.85625) (end 118.26875 89.69375) (width 0.254) (layer "B.Cu") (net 8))
 (segment (start 107.9625 92.0875) (end 109.5375 93.6625) (width 0.254) (layer "B.Cu") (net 8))
 (segment (start 123.88125 87.25625) (end 124.13125 87.25625) (width 0.254) (layer "B.Cu") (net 8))
 (segment (start 131.7625 96.68125) (end 130.84375 97.6) (width 0.254) (layer "B.Cu") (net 8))
 (segment (start 119.121772 92.7125) (end 121.43125 95.021978) (width 0.254) (layer "B.Cu") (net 8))
 (segment (start 99.21875 117.475) (end 99.21875 110.33125) (width 0.254) (layer "B.Cu") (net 8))
 (segment (start 126.05 110.33125) (end 129.225 113.50625) (width 0.254) (layer "B.Cu") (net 8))
 (segment (start 117.63125 89.05625) (end 116.68125 88.10625) (width 0.254) (layer "B.Cu") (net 8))
 (segment (start 109.5375 102.39375) (end 115.09375 102.39375) (width 0.254) (layer "B.Cu") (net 8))
 (segment (start 127.79375 87.15625) (end 127.69375 87.25625) (width 0.254) (layer "B.Cu") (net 8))
 (segment (start 121.93125 88.95625) (end 122.18125 88.95625) (width 0.254) (layer "B.Cu") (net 8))
 (segment (start 130.84375 97.6) (end 128.73125 97.6) (width 0.254) (layer "B.Cu") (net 8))
 (segment (start 127.03125 97.6) (end 128.73125 97.6) (width 0.254) (layer "B.Cu") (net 8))
 (segment (start 118.26875 89.69375) (end 118.26875 89.05625) (width 0.254) (layer "B.Cu") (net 8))
 (segment (start 118.2625 102.4) (end 117.33125 102.4) (width 0.254) (layer "B.Cu") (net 8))
 (segment (start 99.48125 117.7375) (end 99.21875 117.475) (width 0.254) (layer "B.Cu") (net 8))
 (segment (start 126.23125 100.0375) (end 126.23125 107.3) (width 0.254) (layer "B.Cu") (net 8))
 (segment (start 129.225 113.50625) (end 132.55625 113.50625) (width 0.254) (layer "B.Cu") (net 8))
 (segment (start 121.43125 95.021978) (end 121.43125 95.9) (width 0.254) (layer "B.Cu") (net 8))
 (segment (start 124.13125 88.95625) (end 127.69375 88.95625) (width 0.254) (layer "B.Cu") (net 12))
 (segment (start 123.03125 95.9) (end 123.03125 92.075) (width 0.254) (layer "B.Cu") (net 12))
 (segment (start 127.69375 88.95625) (end 127.79375 89.05625) (width 0.254) (layer "B.Cu") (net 12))
 (segment (start 123.825 92.075) (end 124.13125 91.76875) (width 0.254) (layer "B.Cu") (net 12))
 (segment (start 124.13125 91.76875) (end 124.13125 88.95625) (width 0.254) (layer "B.Cu") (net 12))
 (segment (start 123.03125 92.075) (end 123.825 92.075) (width 0.254) (layer "B.Cu") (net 12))
 (segment (start 121.83125 87.25625) (end 120.65 88.4375) (width 0.254) (layer "B.Cu") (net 10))
 (segment (start 118.36875 87.25625) (end 121.93125 87.25625) (width 0.254) (layer "B.Cu") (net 10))
 (segment (start 120.65 88.4375) (end 120.65 90.4875) (width 0.254) (layer "B.Cu") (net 10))
 (segment (start 120.65 90.4875) (end 122.2375 92.075) (width 0.254) (layer "B.Cu") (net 10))
 (segment (start 118.26875 87.15625) (end 118.36875 87.25625) (width 0.254) (layer "B.Cu") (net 10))
 (segment (start 121.93125 87.25625) (end 121.83125 87.25625) (width 0.254) (layer "B.Cu") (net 10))
 (segment (start 122.2375 92.075) (end 122.23125 92.08125) (width 0.254) (layer "B.Cu") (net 10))
 (segment (start 122.23125 92.08125) (end 122.23125 95.9) (width 0.254) (layer "B.Cu") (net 10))
 (segment (start 113.78975 99.0625) (end 113.50625 99.0625) (width 0.254) (layer "B.Cu") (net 23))
 (segment (start 117.33125 101.6) (end 116.32725 101.6) (width 0.254) (layer "B.Cu") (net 23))
 (segment (start 116.32725 101.6) (end 113.78975 99.0625) (width 0.254) (layer "B.Cu") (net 23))
 (segment (start 131.7625 110.33125) (end 129.38125 110.33125) (width 0.254) (layer "F.Cu") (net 11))
 (segment (start 114.3 106.3625) (end 118.26875 110.33125) (width 0.254) (layer "F.Cu") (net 11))
 (segment (start 115.796246 104.866254) (end 115.796246 100.041568) (width 0.254) (layer "F.Cu") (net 11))
 (segment (start 115.796246 100.041568) (end 115.796246 95.158746) (width 0.254) (layer "F.Cu") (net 11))
 (segment (start 133.35 108.74375) (end 131.7625 110.33125) (width 0.254) (layer "F.Cu") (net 11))
 (segment (start 114.3 106.3625) (end 115.796246 104.866254) (width 0.254) (layer "F.Cu") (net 11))
 (segment (start 115.796246 95.158746) (end 113.50625 92.86875) (width 0.254) (layer "F.Cu") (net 11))
 (segment (start 133.35 98.425) (end 133.35 108.74375) (width 0.254) (layer "F.Cu") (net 11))
 (segment (start 118.26875 110.33125) (end 129.38125 110.33125) (width 0.254) (layer "F.Cu") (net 11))
 (via (at 114.3 106.3625) (size 0.8) (drill 0.4) (layers "F.Cu" "B.Cu") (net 11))
 (via (at 115.796246 100.041568) (size 0.8) (drill 0.4) (layers "F.Cu" "B.Cu") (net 11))
 (via (at 129.38125 110.33125) (size 0.8) (drill 0.4) (layers "F.Cu" "B.Cu") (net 11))
 (via (at 133.35 98.425) (size 0.8) (drill 0.4) (layers "F.Cu" "B.Cu") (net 11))
 (via (at 113.50625 92.86875) (size 0.8) (drill 0.4) (layers "F.Cu" "B.Cu") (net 11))
 (segment (start 118.26875 108.74375) (end 119.03125 107.98125) (width 0.254) (layer "B.Cu") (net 11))
 (segment (start 119.03125 107.98125) (end 119.03125 107.3) (width 0.254) (layer "B.Cu") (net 11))
 (segment (start 100.80625 104.5875) (end 104.0125 107.79375) (width 0.254) (layer "B.Cu") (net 11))
 (segment (start 112.0375 92.86875) (end 111.91875 92.75) (width 0.254) (layer "B.Cu") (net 11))
 (segment (start 113.50625 92.86875) (end 112.0375 92.86875) (width 0.254) (layer "B.Cu") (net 11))
 (segment (start 115.8875 107.15625) (end 115.25 107.79375) (width 0.254) (layer "B.Cu") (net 11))
 (segment (start 115.8875 105.23975) (end 116.32725 104.8) (width 0.254) (layer "B.Cu") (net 11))
 (segment (start 127.95 110.33125) (end 127.95 108.9) (width 0.254) (layer "B.Cu") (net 11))
 (segment (start 120.63125 95.021978) (end 120.63125 95.9) (width 0.254) (layer "B.Cu") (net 11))
 (segment (start 116.68125 93.6625) (end 119.271772 93.6625) (width 0.254) (layer "B.Cu") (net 11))
 (segment (start 115.09375 94.6125) (end 115.73125 94.6125) (width 0.254) (layer "B.Cu") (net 11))
 (segment (start 115.8875 108.74375) (end 118.26875 108.74375) (width 0.254) (layer "B.Cu") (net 11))
 (segment (start 119.271772 93.6625) (end 120.63125 95.021978) (width 0.254) (layer "B.Cu") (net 11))
 (segment (start 131.7625 98.58125) (end 131.58125 98.4) (width 0.254) (layer "B.Cu") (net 11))
 (segment (start 116.32725 104.8) (end 117.33125 104.8) (width 0.254) (layer "B.Cu") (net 11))
 (segment (start 131.58125 98.4) (end 128.73125 98.4) (width 0.254) (layer "B.Cu") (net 11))
 (segment (start 115.73125 94.6125) (end 116.68125 93.6625) (width 0.254) (layer "B.Cu") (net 11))
 (segment (start 104.0125 107.79375) (end 114.3 107.79375) (width 0.254) (layer "B.Cu") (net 11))
 (segment (start 114.9375 107.79375) (end 115.8875 108.74375) (width 0.254) (layer "B.Cu") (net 11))
 (segment (start 127.95 108.9) (end 127.03125 107.98125) (width 0.254) (layer "B.Cu") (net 11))
 (segment (start 129.38125 110.33125) (end 127.95 110.33125) (width 0.254) (layer "B.Cu") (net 11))
 (segment (start 115.25 107.79375) (end 114.3 107.79375) (width 0.254) (layer "B.Cu") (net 11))
 (segment (start 111.91875 92.75) (end 113.78125 94.6125) (width 0.254) (layer "B.Cu") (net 11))
 (segment (start 131.7625 98.58125) (end 133.19375 98.58125) (width 0.254) (layer "B.Cu") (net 11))
 (segment (start 117.33125 100.8) (end 116.554678 100.8) (width 0.254) (layer "B.Cu") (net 11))
 (segment (start 133.19375 98.58125) (end 133.35 98.425) (width 0.254) (layer "B.Cu") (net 11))
 (segment (start 115.8875 107.15625) (end 115.8875 105.23975) (width 0.254) (layer "B.Cu") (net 11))
 (segment (start 113.78125 94.6125) (end 115.09375 94.6125) (width 0.254) (layer "B.Cu") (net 11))
 (segment (start 116.554678 100.8) (end 115.796246 100.041568) (width 0.254) (layer "B.Cu") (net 11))
 (segment (start 114.3 107.79375) (end 114.9375 107.79375) (width 0.254) (layer "B.Cu") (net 11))
 (segment (start 127.03125 107.98125) (end 127.03125 107.3) (width 0.254) (layer "B.Cu") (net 11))
 (segment (start 114.3 107.79375) (end 114.3 106.3625) (width 0.254) (layer "B.Cu") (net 11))
 (segment (start 104.7625 91.29375) (end 100.80625 95.25) (width 0.254) (layer "B.Cu") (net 17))
 (segment (start 104.7625 90.225) (end 104.7625 91.29375) (width 0.254) (layer "B.Cu") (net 17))
 (segment (start 100.80625 95.25) (end 100.80625 101.7875) (width 0.254) (layer "B.Cu") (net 17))
 (segment (start 110.33125 112.7125) (end 109.00625 114.0375) (width 0.254) (layer "F.Cu") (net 13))
 (segment (start 110.33125 94.45625) (end 110.33125 112.7125) (width 0.254) (layer "F.Cu") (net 13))
 (via (at 109.00625 114.0375) (size 0.8) (drill 0.4) (layers "F.Cu" "B.Cu") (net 13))
 (via (at 110.33125 94.45625) (size 0.8) (drill 0.4) (layers "F.Cu" "B.Cu") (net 13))
 (segment (start 119.85625 96.04375) (end 119.83125 96.01875) (width 0.254) (layer "B.Cu") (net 13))
 (segment (start 110.45 94.575) (end 110.33125 94.45625) (width 0.254) (layer "B.Cu") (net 13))
 (segment (start 117.901511 94.823489) (end 119.632761 94.823489) (width 0.254) (layer "B.Cu") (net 13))
 (segment (start 119.83125 96.01875) (end 119.83125 95.9) (width 0.254) (layer "B.Cu") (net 13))
 (segment (start 116.68125 96.04375) (end 117.901511 94.823489) (width 0.254) (layer "B.Cu") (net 13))
 (segment (start 108.48125 114.0375) (end 109.00625 114.0375) (width 0.254) (layer "B.Cu") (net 13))
 (segment (start 111.91875 94.575) (end 113.3875 96.04375) (width 0.254) (layer "B.Cu") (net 13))
 (segment (start 111.91875 94.575) (end 112.0375 94.575) (width 0.254) (layer "B.Cu") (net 13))
 (segment (start 119.85625 95.046978) (end 119.85625 96.04375) (width 0.254) (layer "B.Cu") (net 13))
 (segment (start 111.91875 94.575) (end 110.45 94.575) (width 0.254) (layer "B.Cu") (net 13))
 (segment (start 113.3875 96.04375) (end 116.68125 96.04375) (width 0.254) (layer "B.Cu") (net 13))
 (segment (start 119.632761 94.823489) (end 119.85625 95.046978) (width 0.254) (layer "B.Cu") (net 13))
 (segment (start 107.08125 114.0375) (end 108.48125 114.0375) (width 0.254) (layer "B.Cu") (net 13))
 (segment (start 106.3625 92.75) (end 107.95 94.3375) (width 0.2) (layer "B.Cu") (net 15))
 (segment (start 106.3625 90.225) (end 106.3625 92.75) (width 0.2) (layer "B.Cu") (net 15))
 (segment (start 107.95 103.1875) (end 107.9625 103.2) (width 0.254) (layer "B.Cu") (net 16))
 (segment (start 107.9625 103.2) (end 117.33125 103.2) (width 0.254) (layer "B.Cu") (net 16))
 (segment (start 107.95 96.1625) (end 107.95 103.1875) (width 0.254) (layer "B.Cu") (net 16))
 (segment (start 105.5625 93.55) (end 104.775 94.3375) (width 0.2) (layer "B.Cu") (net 18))
 (segment (start 105.5625 90.225) (end 105.5625 93.55) (width 0.2) (layer "B.Cu") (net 18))
 (segment (start 104.775 96.1625) (end 104.775 103.98125) (width 0.254) (layer "B.Cu") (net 19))
 (segment (start 104.775 103.98125) (end 104.79375 104) (width 0.254) (layer "B.Cu") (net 19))
 (segment (start 104.79375 104) (end 117.33125 104) (width 0.254) (layer "B.Cu") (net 19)))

